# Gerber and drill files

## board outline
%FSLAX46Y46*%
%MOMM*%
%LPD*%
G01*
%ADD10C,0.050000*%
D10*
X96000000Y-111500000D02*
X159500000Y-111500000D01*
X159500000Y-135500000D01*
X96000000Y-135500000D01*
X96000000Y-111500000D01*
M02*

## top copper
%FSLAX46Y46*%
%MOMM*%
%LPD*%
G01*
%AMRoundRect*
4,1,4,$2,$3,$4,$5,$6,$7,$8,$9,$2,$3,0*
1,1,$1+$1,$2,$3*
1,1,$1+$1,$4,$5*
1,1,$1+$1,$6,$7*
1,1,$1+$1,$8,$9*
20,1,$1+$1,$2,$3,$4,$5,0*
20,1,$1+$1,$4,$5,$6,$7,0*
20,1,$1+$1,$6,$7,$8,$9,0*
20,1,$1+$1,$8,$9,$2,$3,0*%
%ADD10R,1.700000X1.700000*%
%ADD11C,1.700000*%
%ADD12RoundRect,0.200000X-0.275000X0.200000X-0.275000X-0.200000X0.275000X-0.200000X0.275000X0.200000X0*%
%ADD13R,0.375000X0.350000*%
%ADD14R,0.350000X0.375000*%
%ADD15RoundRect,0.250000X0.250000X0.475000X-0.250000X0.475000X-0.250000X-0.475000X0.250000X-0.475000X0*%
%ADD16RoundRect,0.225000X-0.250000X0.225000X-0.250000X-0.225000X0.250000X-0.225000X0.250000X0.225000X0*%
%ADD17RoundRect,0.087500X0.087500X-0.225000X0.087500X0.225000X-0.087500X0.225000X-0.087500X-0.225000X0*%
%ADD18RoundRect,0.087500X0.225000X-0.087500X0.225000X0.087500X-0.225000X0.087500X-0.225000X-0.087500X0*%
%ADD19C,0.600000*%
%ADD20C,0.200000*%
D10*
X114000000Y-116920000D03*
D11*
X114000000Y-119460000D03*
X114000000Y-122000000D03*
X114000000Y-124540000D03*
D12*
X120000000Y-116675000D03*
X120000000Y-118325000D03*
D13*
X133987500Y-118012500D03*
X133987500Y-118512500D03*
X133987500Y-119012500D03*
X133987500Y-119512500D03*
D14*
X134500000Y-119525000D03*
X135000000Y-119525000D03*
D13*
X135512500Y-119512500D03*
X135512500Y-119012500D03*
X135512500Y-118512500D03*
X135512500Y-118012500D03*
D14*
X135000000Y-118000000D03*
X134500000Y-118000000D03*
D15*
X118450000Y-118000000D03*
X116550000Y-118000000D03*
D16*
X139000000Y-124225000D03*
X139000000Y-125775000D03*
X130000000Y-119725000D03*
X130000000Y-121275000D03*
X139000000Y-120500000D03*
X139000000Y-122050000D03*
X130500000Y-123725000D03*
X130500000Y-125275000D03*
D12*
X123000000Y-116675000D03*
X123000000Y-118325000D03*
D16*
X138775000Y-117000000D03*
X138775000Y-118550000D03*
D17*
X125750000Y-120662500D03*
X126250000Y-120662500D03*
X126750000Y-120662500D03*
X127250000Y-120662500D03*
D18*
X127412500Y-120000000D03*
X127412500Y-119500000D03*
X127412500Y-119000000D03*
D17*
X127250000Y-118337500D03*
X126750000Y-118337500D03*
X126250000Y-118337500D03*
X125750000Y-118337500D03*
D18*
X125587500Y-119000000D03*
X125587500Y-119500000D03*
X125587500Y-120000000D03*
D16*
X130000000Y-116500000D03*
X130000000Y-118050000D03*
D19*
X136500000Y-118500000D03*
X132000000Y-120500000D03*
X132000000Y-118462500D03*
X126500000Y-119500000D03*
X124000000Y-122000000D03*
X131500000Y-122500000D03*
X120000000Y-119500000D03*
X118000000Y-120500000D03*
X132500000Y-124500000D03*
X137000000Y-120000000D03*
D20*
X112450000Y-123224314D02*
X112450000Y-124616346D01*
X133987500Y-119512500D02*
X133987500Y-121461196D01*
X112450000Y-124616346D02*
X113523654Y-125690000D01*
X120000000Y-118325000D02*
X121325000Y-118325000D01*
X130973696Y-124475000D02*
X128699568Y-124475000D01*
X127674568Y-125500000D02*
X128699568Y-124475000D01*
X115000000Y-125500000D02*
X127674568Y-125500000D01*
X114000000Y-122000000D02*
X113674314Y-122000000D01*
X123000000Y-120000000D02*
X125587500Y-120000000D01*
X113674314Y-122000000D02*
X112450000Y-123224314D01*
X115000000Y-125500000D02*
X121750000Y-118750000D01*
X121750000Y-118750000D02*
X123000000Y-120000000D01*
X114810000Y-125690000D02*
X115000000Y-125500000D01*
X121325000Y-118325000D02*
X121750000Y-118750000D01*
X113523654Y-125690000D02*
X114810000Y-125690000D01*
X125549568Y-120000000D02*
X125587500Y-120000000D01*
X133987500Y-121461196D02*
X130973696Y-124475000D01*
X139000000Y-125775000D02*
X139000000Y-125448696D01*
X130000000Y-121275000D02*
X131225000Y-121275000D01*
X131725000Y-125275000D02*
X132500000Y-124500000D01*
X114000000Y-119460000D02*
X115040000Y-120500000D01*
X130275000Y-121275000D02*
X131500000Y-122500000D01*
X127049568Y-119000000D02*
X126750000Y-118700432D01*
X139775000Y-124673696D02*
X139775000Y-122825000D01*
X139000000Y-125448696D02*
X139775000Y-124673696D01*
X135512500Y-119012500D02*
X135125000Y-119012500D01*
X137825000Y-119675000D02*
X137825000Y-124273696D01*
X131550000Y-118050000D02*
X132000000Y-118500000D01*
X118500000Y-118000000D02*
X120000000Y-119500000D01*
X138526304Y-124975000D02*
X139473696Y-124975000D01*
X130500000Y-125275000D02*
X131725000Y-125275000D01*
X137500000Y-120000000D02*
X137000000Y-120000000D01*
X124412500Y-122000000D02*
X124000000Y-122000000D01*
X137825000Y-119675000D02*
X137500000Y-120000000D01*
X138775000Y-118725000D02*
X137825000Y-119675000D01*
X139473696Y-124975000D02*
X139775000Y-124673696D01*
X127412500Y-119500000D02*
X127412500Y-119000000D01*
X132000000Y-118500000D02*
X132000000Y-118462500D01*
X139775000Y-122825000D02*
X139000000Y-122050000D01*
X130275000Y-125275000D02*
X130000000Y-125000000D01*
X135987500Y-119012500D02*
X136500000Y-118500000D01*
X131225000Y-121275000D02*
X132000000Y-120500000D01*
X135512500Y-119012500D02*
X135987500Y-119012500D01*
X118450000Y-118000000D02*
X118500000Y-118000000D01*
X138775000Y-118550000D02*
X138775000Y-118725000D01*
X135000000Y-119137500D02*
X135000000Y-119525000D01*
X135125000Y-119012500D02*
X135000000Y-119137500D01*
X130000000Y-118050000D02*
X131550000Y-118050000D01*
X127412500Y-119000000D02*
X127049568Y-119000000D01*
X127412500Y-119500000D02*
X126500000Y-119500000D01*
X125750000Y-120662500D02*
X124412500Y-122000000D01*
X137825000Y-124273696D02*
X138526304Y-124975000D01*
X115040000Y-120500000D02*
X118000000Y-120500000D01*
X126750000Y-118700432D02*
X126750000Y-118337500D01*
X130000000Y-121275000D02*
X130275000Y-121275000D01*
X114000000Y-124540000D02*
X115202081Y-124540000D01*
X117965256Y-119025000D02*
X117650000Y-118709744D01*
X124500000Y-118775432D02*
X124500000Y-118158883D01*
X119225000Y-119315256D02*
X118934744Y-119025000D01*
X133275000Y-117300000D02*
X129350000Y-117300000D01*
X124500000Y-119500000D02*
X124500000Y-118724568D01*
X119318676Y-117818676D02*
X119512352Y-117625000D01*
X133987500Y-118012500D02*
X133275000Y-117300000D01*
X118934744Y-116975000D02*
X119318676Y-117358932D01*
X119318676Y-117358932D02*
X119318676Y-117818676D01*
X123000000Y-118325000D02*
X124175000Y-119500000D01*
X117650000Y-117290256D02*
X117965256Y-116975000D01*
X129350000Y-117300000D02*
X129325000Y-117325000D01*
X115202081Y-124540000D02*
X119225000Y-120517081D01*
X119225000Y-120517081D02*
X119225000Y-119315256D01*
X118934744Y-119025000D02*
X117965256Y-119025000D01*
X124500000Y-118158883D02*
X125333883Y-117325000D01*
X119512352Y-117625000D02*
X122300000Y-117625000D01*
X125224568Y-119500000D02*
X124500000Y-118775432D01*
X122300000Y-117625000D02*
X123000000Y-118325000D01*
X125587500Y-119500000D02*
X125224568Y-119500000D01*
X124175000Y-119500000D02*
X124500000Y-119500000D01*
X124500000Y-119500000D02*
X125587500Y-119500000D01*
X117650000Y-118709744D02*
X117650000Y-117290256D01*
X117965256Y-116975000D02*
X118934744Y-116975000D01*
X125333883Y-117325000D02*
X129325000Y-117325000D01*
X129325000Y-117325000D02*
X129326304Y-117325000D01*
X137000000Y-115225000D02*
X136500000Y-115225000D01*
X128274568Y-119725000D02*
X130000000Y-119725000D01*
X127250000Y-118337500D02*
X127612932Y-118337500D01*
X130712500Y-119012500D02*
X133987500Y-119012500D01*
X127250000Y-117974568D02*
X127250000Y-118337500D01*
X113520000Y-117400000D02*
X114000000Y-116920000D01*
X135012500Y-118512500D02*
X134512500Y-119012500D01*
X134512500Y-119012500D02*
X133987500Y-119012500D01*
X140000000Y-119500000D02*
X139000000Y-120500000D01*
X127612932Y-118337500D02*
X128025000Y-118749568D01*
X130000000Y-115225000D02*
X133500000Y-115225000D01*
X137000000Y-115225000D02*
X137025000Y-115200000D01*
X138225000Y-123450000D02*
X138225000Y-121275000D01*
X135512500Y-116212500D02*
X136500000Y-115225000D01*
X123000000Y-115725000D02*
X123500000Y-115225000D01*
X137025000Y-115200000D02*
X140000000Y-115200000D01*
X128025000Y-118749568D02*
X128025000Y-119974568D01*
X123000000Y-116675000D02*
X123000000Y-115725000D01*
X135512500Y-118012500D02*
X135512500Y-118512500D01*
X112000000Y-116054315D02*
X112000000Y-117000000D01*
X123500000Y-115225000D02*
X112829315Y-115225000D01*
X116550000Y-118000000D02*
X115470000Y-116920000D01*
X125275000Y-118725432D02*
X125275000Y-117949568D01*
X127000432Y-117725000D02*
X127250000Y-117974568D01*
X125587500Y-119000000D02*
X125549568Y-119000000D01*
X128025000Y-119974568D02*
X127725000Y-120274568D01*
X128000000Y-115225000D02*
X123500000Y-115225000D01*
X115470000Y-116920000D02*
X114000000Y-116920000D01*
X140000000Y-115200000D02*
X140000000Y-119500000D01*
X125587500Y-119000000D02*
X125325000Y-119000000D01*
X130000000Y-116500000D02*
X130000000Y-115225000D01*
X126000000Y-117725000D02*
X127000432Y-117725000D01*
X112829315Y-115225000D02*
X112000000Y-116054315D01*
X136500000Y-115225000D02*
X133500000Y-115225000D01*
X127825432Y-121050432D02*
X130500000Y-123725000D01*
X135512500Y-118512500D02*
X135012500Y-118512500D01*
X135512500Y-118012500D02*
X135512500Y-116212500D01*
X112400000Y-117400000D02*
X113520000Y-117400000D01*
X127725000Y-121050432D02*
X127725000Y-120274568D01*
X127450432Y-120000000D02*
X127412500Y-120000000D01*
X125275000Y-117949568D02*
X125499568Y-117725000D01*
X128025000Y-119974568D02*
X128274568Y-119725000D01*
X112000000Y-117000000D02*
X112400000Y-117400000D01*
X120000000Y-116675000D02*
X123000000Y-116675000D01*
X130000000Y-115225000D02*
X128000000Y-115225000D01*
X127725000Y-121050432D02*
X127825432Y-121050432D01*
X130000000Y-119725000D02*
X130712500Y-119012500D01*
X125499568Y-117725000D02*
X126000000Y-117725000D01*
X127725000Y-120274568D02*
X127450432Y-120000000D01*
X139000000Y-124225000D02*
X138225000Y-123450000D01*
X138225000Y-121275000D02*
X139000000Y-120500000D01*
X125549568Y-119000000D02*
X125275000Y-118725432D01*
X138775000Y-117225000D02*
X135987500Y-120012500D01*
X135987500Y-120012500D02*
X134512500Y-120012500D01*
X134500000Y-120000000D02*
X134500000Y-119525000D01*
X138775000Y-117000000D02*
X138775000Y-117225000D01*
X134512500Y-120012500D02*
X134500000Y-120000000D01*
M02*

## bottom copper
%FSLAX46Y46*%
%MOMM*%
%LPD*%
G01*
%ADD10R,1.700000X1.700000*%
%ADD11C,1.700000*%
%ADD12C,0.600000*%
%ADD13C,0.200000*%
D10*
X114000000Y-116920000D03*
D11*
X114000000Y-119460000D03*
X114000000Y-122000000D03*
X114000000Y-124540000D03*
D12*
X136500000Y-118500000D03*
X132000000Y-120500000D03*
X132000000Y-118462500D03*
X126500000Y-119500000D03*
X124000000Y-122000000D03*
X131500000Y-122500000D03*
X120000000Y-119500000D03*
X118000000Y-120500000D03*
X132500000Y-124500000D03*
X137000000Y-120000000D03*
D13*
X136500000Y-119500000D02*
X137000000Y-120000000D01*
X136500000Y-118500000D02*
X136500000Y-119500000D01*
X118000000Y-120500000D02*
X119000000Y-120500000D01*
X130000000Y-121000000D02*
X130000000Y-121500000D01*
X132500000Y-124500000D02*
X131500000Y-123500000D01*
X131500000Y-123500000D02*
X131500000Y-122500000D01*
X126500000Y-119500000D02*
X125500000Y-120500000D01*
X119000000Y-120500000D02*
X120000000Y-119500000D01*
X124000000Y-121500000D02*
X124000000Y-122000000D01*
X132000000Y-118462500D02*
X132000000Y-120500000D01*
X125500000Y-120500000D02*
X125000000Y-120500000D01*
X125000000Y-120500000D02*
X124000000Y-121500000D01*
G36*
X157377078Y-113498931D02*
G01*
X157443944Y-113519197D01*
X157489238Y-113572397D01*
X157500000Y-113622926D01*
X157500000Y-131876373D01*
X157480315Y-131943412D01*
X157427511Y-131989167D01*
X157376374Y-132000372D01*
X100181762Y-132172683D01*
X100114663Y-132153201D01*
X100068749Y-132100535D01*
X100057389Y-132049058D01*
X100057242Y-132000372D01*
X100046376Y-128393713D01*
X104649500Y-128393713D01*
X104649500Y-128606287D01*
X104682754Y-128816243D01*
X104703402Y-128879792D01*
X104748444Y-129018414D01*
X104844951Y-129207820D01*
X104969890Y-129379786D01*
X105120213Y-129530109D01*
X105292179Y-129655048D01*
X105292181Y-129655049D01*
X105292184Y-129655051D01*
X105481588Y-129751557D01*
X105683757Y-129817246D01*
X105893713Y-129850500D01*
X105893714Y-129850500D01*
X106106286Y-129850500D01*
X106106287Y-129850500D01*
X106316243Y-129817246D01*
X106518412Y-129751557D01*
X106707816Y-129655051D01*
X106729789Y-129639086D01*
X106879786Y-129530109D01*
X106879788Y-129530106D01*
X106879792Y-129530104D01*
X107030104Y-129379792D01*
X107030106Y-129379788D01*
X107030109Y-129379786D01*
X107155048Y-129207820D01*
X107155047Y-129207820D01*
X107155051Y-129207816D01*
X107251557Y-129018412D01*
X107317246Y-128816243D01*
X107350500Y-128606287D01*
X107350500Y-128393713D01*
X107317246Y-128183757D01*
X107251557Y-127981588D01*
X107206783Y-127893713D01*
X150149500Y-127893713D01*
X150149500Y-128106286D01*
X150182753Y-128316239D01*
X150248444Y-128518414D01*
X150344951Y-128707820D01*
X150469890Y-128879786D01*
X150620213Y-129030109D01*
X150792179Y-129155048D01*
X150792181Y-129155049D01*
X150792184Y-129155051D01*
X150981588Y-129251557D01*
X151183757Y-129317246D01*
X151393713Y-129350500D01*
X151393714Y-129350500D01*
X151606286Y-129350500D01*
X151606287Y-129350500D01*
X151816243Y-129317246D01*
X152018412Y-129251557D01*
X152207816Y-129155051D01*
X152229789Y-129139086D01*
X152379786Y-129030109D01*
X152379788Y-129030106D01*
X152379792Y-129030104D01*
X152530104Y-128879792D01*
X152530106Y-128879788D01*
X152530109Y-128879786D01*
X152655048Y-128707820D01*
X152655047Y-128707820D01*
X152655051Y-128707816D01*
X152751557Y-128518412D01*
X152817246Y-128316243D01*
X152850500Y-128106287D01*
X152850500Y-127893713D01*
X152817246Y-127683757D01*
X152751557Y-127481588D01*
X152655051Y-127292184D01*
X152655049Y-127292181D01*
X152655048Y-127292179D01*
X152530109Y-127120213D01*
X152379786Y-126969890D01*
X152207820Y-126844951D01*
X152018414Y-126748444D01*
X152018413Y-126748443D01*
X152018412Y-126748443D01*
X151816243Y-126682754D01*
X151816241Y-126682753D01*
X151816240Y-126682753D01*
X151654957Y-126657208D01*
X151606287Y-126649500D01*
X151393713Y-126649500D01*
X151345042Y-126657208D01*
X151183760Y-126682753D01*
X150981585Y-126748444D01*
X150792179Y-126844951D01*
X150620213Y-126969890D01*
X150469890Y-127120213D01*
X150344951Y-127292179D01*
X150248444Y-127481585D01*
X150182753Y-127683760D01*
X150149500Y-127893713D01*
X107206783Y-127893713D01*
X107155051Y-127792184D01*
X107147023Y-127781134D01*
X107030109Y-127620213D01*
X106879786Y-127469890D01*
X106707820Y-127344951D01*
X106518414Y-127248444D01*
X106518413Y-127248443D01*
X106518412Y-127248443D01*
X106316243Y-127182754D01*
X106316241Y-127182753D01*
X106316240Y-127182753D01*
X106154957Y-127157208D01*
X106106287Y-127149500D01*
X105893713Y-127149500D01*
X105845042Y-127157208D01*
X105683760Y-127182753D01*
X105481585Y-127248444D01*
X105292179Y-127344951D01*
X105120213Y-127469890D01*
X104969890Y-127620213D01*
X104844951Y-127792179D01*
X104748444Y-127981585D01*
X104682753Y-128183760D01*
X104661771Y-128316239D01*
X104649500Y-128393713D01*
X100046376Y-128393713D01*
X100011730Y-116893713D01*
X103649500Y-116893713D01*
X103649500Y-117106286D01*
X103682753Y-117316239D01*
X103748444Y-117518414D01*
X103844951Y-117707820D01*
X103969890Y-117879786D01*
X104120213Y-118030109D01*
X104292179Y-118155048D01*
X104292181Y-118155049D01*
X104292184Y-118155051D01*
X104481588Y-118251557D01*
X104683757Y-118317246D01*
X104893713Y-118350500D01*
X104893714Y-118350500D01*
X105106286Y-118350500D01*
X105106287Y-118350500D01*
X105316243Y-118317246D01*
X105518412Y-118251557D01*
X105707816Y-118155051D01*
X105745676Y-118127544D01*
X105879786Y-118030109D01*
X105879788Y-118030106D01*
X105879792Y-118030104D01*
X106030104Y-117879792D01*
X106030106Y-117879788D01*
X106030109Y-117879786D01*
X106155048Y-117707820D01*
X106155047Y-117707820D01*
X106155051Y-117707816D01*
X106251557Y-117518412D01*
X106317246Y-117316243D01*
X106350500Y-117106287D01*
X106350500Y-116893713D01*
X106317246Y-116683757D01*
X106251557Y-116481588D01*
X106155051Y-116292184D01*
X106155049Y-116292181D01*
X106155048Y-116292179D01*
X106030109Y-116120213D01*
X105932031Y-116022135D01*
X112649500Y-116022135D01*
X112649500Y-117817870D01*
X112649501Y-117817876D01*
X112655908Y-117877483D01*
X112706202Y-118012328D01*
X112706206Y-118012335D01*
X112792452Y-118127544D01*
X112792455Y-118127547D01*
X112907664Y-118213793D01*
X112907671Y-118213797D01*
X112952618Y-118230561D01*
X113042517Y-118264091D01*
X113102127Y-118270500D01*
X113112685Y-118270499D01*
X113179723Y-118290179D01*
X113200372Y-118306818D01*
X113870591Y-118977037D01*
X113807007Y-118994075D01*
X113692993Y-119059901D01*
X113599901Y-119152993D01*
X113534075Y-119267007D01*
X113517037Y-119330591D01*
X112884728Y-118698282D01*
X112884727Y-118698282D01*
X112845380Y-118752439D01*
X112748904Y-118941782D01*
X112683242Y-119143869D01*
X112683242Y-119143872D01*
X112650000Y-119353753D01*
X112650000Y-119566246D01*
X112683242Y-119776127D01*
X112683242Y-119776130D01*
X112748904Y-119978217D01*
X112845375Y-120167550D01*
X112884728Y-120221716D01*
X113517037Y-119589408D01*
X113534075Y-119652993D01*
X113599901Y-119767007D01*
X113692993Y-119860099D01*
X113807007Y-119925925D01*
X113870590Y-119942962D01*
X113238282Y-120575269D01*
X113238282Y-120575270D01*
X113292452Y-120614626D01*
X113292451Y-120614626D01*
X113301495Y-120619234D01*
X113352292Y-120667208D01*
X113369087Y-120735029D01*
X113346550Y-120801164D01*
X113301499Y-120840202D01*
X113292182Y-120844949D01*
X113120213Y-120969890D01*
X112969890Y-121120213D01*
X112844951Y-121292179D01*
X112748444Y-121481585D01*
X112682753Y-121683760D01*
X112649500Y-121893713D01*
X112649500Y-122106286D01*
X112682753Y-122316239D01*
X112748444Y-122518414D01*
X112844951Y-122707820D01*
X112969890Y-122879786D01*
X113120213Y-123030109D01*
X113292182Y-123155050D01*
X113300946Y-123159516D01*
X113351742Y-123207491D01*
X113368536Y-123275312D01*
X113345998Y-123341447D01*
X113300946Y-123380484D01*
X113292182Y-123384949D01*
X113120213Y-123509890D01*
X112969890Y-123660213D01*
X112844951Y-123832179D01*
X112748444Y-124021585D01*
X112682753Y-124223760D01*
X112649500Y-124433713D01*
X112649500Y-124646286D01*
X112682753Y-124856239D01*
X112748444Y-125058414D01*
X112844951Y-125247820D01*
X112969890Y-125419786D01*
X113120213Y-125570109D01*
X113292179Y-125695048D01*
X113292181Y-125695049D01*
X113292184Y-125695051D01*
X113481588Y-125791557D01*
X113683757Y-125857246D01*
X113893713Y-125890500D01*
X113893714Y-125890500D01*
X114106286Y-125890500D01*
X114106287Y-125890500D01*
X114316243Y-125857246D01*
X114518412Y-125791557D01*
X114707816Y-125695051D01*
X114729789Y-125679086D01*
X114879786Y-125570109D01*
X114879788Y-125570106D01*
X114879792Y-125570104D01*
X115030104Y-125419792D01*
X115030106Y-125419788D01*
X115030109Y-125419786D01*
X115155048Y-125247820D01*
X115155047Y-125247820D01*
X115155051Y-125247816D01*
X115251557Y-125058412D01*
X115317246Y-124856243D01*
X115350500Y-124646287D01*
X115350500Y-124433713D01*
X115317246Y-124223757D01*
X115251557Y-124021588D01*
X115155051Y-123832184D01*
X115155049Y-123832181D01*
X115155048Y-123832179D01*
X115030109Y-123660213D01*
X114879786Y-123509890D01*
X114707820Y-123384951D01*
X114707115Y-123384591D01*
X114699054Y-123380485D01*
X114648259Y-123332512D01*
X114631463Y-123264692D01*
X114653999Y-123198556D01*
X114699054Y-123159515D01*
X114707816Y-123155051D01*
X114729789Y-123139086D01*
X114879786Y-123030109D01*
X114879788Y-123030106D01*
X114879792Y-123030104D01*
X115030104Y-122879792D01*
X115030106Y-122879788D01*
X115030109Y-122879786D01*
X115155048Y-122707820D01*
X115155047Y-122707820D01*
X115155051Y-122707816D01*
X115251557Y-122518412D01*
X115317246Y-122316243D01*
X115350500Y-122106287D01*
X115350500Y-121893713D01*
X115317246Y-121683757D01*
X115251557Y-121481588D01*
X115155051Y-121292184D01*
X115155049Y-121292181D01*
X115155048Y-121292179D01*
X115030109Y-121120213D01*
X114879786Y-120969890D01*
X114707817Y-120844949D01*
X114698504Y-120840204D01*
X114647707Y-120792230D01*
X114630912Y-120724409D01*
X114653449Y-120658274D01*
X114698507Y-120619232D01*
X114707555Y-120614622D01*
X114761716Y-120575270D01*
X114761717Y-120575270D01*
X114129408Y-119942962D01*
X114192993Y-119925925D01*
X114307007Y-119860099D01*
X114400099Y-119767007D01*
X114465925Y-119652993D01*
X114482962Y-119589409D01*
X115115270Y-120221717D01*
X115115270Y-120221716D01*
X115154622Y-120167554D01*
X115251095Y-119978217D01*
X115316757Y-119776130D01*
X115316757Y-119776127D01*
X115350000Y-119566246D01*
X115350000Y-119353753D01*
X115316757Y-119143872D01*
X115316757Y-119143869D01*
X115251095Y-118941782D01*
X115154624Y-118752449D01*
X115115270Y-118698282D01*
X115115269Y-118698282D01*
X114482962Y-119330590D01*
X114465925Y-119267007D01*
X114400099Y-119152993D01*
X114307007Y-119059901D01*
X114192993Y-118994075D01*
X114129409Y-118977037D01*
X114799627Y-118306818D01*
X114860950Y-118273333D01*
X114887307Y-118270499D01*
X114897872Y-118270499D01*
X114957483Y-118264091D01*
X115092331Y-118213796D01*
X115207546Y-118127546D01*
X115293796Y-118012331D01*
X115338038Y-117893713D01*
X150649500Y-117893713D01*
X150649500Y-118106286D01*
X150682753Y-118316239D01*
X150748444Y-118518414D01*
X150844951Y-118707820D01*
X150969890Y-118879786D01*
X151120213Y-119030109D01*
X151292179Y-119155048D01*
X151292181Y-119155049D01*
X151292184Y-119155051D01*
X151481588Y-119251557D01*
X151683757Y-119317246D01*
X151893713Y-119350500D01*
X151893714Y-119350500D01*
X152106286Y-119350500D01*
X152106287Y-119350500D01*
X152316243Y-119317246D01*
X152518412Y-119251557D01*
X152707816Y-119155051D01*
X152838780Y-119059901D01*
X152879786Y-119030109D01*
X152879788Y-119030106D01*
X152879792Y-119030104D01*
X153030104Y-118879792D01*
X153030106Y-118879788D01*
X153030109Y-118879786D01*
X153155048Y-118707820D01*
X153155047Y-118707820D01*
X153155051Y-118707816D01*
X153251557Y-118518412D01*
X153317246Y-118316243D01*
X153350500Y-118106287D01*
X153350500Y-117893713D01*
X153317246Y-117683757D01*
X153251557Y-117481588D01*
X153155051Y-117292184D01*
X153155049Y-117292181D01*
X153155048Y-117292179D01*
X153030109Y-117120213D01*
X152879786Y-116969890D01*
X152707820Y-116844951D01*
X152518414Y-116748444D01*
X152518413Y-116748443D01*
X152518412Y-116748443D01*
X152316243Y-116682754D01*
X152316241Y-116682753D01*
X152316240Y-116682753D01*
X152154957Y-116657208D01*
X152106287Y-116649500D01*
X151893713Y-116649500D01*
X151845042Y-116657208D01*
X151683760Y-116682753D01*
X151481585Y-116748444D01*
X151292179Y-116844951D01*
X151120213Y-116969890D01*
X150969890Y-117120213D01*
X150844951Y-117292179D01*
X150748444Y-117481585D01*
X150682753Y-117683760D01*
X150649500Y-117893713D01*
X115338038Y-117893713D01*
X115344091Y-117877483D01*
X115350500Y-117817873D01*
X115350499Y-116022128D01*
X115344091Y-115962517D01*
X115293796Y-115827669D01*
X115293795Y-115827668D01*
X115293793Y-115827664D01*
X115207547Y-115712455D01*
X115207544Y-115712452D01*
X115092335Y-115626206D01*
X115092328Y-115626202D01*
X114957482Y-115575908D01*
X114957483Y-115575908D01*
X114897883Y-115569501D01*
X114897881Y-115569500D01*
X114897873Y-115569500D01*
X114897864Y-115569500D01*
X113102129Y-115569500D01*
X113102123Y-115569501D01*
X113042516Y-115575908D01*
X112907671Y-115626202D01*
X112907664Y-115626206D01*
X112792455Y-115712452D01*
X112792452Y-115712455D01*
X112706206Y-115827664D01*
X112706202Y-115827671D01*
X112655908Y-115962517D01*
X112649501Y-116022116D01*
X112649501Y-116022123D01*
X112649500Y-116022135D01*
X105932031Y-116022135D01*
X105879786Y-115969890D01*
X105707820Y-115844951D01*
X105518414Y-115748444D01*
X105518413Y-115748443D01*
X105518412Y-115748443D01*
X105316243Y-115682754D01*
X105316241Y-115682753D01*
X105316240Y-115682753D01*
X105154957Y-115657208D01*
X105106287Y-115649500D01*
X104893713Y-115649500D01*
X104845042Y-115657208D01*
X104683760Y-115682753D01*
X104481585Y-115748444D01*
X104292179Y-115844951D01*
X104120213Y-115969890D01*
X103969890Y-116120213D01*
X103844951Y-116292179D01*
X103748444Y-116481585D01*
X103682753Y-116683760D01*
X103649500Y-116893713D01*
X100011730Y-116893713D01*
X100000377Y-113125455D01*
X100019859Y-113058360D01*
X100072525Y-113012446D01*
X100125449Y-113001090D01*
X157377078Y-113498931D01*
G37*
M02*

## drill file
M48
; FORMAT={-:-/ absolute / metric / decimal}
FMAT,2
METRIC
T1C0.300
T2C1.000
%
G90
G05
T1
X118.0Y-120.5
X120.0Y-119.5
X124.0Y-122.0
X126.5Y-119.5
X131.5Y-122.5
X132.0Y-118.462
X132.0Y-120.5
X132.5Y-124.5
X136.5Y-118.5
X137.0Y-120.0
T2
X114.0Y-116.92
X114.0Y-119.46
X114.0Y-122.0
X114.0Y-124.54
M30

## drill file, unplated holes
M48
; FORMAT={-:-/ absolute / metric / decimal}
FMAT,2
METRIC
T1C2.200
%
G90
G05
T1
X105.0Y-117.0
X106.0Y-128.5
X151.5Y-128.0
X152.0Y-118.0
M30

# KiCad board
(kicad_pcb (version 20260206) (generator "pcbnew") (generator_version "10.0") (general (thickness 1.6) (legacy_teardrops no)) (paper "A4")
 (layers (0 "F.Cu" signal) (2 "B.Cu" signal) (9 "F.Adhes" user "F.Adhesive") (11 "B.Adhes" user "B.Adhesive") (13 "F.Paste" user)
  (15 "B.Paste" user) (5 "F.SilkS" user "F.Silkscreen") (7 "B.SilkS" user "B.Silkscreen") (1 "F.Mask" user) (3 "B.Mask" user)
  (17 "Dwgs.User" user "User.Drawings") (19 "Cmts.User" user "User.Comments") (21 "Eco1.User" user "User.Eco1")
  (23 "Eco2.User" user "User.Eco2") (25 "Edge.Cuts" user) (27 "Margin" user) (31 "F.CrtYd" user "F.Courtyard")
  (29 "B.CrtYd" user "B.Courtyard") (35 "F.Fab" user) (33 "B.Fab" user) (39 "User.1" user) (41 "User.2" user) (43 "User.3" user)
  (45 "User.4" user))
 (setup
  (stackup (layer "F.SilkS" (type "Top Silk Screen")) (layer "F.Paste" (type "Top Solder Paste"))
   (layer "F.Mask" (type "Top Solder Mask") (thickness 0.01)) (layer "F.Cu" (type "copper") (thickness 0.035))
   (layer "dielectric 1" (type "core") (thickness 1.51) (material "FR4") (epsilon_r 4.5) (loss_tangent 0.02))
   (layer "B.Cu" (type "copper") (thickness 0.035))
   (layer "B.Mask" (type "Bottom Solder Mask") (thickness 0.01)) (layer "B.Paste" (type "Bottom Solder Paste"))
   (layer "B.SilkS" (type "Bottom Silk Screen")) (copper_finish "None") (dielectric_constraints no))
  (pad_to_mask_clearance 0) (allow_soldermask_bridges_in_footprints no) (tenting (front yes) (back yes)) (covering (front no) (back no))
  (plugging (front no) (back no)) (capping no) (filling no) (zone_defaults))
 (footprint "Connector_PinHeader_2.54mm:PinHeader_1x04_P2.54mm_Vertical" (layer "F.Cu") (at 114 116.92)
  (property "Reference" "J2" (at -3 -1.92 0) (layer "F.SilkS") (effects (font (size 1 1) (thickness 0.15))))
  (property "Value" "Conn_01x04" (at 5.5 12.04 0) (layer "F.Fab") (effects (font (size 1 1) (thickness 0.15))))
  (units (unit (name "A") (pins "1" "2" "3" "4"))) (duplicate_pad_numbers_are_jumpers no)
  (pad "1" thru_hole rect (at 0 0) (size 1.7 1.7) (drill 1) (layers "*.Cu" "*.Mask") (remove_unused_layers no) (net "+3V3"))
  (pad "2" thru_hole circle (at 0 2.54) (size 1.7 1.7) (drill 1) (layers "*.Cu" "*.Mask") (remove_unused_layers no) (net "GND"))
  (pad "3" thru_hole circle (at 0 5.08) (size 1.7 1.7) (drill 1) (layers "*.Cu" "*.Mask") (remove_unused_layers no) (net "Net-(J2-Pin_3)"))
  (pad "4" thru_hole circle (at 0 7.62) (size 1.7 1.7) (drill 1) (layers "*.Cu" "*.Mask") (remove_unused_layers no) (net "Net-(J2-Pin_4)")))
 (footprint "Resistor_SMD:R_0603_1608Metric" (layer "F.Cu") (at 120 117.5 -90)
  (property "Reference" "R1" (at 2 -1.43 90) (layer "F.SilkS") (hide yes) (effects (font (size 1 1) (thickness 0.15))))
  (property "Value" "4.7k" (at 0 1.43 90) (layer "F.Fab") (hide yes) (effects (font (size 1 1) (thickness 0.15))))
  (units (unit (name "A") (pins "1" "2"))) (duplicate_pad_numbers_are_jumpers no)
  (pad "1" smd roundrect (at -0.825 0 270) (size 0.8 0.95) (layers "F.Cu" "F.Mask" "F.Paste") (roundrect_rratio 0.25) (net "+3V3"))
  (pad "2" smd roundrect (at 0.825 0 270) (size 0.8 0.95) (layers "F.Cu" "F.Mask" "F.Paste") (roundrect_rratio 0.25) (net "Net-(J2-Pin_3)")))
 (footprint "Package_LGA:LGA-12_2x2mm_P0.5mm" (layer "F.Cu") (at 134.75 118.7625)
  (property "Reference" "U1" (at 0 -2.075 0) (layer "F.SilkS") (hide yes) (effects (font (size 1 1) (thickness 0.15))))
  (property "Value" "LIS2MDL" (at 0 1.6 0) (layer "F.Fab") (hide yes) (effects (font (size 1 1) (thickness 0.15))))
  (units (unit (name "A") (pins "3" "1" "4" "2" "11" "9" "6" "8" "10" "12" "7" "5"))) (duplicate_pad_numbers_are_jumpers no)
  (pad "1" smd rect (at -0.7625 -0.75) (size 0.375 0.35) (layers "F.Cu" "F.Mask" "F.Paste") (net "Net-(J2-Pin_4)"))
  (pad "2" smd rect (at -0.7625 -0.25) (size 0.375 0.35) (layers "F.Cu" "F.Mask" "F.Paste") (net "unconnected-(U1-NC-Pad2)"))
  (pad "3" smd rect (at -0.7625 0.25) (size 0.375 0.35) (layers "F.Cu" "F.Mask" "F.Paste") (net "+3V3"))
  (pad "4" smd rect (at -0.7625 0.75) (size 0.375 0.35) (layers "F.Cu" "F.Mask" "F.Paste") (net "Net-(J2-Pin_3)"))
  (pad "5" smd rect (at -0.25 0.7625 90) (size 0.375 0.35) (layers "F.Cu" "F.Mask" "F.Paste") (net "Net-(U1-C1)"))
  (pad "6" smd rect (at 0.25 0.7625 90) (size 0.375 0.35) (layers "F.Cu" "F.Mask" "F.Paste") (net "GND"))
  (pad "7" smd rect (at 0.7625 0.75) (size 0.375 0.35) (layers "F.Cu" "F.Mask" "F.Paste") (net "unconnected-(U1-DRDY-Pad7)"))
  (pad "8" smd rect (at 0.7625 0.25) (size 0.375 0.35) (layers "F.Cu" "F.Mask" "F.Paste") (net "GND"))
  (pad "9" smd rect (at 0.7625 -0.25) (size 0.375 0.35) (layers "F.Cu" "F.Mask" "F.Paste") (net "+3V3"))
  (pad "10" smd rect (at 0.7625 -0.75) (size 0.375 0.35) (layers "F.Cu" "F.Mask" "F.Paste") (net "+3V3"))
  (pad "11" smd rect (at 0.25 -0.7625 90) (size 0.375 0.35) (layers "F.Cu" "F.Mask" "F.Paste") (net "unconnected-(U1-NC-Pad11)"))
  (pad "12" smd rect (at -0.25 -0.7625 90) (size 0.375 0.35) (layers "F.Cu" "F.Mask" "F.Paste") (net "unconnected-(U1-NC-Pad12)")))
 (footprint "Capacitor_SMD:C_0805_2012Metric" (layer "F.Cu") (at 117.5 118 180)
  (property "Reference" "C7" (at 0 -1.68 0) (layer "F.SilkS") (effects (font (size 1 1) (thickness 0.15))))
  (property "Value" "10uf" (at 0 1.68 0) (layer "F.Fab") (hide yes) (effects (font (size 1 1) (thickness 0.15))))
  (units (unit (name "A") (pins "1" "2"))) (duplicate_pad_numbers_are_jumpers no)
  (pad "1" smd roundrect (at -0.95 0 180) (size 1 1.45) (layers "F.Cu" "F.Mask" "F.Paste") (roundrect_rratio 0.25) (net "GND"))
  (pad "2" smd roundrect (at 0.95 0 180) (size 1 1.45) (layers "F.Cu" "F.Mask" "F.Paste") (roundrect_rratio 0.25) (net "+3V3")))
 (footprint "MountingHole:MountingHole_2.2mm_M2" (layer "F.Cu") (at 105 117)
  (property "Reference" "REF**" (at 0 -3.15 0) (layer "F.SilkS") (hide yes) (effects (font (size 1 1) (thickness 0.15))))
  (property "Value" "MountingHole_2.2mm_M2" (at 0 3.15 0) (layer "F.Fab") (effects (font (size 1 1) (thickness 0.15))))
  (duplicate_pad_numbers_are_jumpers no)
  (pad "" np_thru_hole circle (at 0 0) (size 2.2 2.2) (drill 2.2) (layers "*.Cu" "*.Mask")))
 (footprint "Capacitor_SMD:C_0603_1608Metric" (layer "F.Cu") (at 139 125 -90)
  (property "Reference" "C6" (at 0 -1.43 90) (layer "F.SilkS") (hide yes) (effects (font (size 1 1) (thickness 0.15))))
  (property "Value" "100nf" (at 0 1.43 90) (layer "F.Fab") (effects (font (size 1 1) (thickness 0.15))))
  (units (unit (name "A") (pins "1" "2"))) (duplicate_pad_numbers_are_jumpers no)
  (pad "1" smd roundrect (at -0.775 0 270) (size 0.9 0.95) (layers "F.Cu" "F.Mask" "F.Paste") (roundrect_rratio 0.25) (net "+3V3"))
  (pad "2" smd roundrect (at 0.775 0 270) (size 0.9 0.95) (layers "F.Cu" "F.Mask" "F.Paste") (roundrect_rratio 0.25) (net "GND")))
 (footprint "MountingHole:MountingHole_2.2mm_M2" (layer "F.Cu") (at 151.5 128)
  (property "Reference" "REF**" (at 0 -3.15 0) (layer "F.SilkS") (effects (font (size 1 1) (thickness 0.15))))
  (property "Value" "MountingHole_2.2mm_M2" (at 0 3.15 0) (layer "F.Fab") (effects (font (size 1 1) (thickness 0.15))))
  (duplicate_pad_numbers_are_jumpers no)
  (pad "" np_thru_hole circle (at 0 0) (size 2.2 2.2) (drill 2.2) (layers "*.Cu" "*.Mask")))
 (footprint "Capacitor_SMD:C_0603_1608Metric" (layer "F.Cu") (at 130 120.5 -90)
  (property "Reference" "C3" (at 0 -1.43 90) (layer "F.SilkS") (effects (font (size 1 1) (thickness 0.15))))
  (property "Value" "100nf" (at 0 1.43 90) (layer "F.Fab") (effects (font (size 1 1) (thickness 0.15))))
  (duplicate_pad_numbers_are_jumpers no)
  (pad "1" smd roundrect (at -0.775 0 270) (size 0.9 0.95) (layers "F.Cu" "F.Mask" "F.Paste") (roundrect_rratio 0.25) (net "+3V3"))
  (pad "2" smd roundrect (at 0.775 0 270) (size 0.9 0.95) (layers "F.Cu" "F.Mask" "F.Paste") (roundrect_rratio 0.25) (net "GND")))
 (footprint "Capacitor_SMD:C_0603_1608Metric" (layer "F.Cu") (at 139 121.275 -90)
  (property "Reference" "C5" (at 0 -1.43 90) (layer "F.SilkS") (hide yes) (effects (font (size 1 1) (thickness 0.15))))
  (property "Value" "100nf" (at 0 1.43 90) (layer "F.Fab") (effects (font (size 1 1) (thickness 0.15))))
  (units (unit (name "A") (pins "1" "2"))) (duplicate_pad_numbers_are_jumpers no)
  (pad "1" smd roundrect (at -0.775 0 270) (size 0.9 0.95) (layers "F.Cu" "F.Mask" "F.Paste") (roundrect_rratio 0.25) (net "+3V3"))
  (pad "2" smd roundrect (at 0.775 0 270) (size 0.9 0.95) (layers "F.Cu" "F.Mask" "F.Paste") (roundrect_rratio 0.25) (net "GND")))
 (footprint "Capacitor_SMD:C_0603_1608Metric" (layer "F.Cu") (at 130.5 124.5 -90)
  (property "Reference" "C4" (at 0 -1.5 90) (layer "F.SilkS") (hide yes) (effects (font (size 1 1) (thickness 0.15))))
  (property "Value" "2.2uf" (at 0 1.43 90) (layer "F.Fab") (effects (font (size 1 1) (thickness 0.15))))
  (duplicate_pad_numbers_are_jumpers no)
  (pad "1" smd roundrect (at -0.775 0 270) (size 0.9 0.95) (layers "F.Cu" "F.Mask" "F.Paste") (roundrect_rratio 0.25) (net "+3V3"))
  (pad "2" smd roundrect (at 0.775 0 270) (size 0.9 0.95) (layers "F.Cu" "F.Mask" "F.Paste") (roundrect_rratio 0.25) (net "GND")))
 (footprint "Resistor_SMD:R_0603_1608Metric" (layer "F.Cu") (at 123 117.5 -90)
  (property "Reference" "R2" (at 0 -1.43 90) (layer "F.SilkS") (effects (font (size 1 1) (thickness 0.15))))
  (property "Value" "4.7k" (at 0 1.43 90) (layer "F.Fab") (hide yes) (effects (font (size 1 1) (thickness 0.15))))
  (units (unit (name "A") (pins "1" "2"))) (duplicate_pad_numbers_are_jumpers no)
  (pad "1" smd roundrect (at -0.825 0 270) (size 0.8 0.95) (layers "F.Cu" "F.Mask" "F.Paste") (roundrect_rratio 0.25) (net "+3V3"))
  (pad "2" smd roundrect (at 0.825 0 270) (size 0.8 0.95) (layers "F.Cu" "F.Mask" "F.Paste") (roundrect_rratio 0.25) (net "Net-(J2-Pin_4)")))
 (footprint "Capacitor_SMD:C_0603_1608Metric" (layer "F.Cu") (at 138.775 117.775 -90)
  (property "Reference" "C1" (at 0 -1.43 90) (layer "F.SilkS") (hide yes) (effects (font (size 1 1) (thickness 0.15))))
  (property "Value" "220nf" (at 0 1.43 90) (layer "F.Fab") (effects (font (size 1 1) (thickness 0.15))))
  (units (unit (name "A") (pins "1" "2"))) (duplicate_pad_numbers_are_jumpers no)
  (pad "1" smd roundrect (at -0.775 0 270) (size 0.9 0.95) (layers "F.Cu" "F.Mask" "F.Paste") (roundrect_rratio 0.25) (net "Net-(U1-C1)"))
  (pad "2" smd roundrect (at 0.775 0 270) (size 0.9 0.95) (layers "F.Cu" "F.Mask" "F.Paste") (roundrect_rratio 0.25) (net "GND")))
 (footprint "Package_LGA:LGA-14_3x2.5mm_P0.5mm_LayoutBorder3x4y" (layer "F.Cu") (at 126.5 119.5 90)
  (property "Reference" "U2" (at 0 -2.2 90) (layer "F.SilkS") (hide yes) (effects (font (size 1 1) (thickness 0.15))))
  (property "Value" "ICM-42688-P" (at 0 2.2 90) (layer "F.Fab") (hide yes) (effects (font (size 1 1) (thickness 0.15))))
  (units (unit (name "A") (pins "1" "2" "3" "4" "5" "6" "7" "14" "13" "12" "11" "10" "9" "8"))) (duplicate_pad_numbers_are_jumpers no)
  (pad "1" smd roundrect (at -1.1625 -0.75 90) (size 0.625 0.35) (layers "F.Cu" "F.Mask" "F.Paste") (roundrect_rratio 0.25) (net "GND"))
  (pad "2" smd roundrect (at -1.1625 -0.25 90) (size 0.625 0.35) (layers "F.Cu" "F.Mask" "F.Paste") (roundrect_rratio 0.25)
   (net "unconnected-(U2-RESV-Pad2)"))
  (pad "3" smd roundrect (at -1.1625 0.25 90) (size 0.625 0.35) (layers "F.Cu" "F.Mask" "F.Paste") (roundrect_rratio 0.25)
   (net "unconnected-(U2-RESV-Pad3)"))
  (pad "4" smd roundrect (at -1.1625 0.75 90) (size 0.625 0.35) (layers "F.Cu" "F.Mask" "F.Paste") (roundrect_rratio 0.25)
   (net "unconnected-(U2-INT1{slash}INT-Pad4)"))
  (pad "5" smd roundrect (at -0.5 0.9125 90) (size 0.35 0.625) (layers "F.Cu" "F.Mask" "F.Paste") (roundrect_rratio 0.25) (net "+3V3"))
  (pad "6" smd roundrect (at 0 0.9125 90) (size 0.35 0.625) (layers "F.Cu" "F.Mask" "F.Paste") (roundrect_rratio 0.25) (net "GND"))
  (pad "7" smd roundrect (at 0.5 0.9125 90) (size 0.35 0.625) (layers "F.Cu" "F.Mask" "F.Paste") (roundrect_rratio 0.25) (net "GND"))
  (pad "8" smd roundrect (at 1.1625 0.75 90) (size 0.625 0.35) (layers "F.Cu" "F.Mask" "F.Paste") (roundrect_rratio 0.25) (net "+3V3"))
  (pad "9" smd roundrect (at 1.1625 0.25 90) (size 0.625 0.35) (layers "F.Cu" "F.Mask" "F.Paste") (roundrect_rratio 0.25) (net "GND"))
  (pad "10" smd roundrect (at 1.1625 -0.25 90) (size 0.625 0.35) (layers "F.Cu" "F.Mask" "F.Paste") (roundrect_rratio 0.25)
   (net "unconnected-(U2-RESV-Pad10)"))
  (pad "11" smd roundrect (at 1.1625 -0.75 90) (size 0.625 0.35) (layers "F.Cu" "F.Mask" "F.Paste") (roundrect_rratio 0.25)
   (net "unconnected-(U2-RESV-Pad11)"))
  (pad "12" smd roundrect (at 0.5 -0.9125 90) (size 0.35 0.625) (layers "F.Cu" "F.Mask" "F.Paste") (roundrect_rratio 0.25) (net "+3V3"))
  (pad "13" smd roundrect (at 0 -0.9125 90) (size 0.35 0.625) (layers "F.Cu" "F.Mask" "F.Paste") (roundrect_rratio 0.25)
   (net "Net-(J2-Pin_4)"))
  (pad "14" smd roundrect (at -0.5 -0.9125 90) (size 0.35 0.625) (layers "F.Cu" "F.Mask" "F.Paste") (roundrect_rratio 0.25)
   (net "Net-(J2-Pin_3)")))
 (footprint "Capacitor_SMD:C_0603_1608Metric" (layer "F.Cu") (at 130 117.275 -90)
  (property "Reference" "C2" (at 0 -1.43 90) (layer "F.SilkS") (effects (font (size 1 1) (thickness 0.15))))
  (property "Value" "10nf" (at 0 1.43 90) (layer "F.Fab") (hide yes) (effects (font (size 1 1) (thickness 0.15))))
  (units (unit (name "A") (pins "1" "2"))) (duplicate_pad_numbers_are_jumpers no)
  (pad "1" smd roundrect (at -0.775 0 270) (size 0.9 0.95) (layers "F.Cu" "F.Mask" "F.Paste") (roundrect_rratio 0.25) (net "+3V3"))
  (pad "2" smd roundrect (at 0.775 0 270) (size 0.9 0.95) (layers "F.Cu" "F.Mask" "F.Paste") (roundrect_rratio 0.25) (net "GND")))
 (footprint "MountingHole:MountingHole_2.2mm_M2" (layer "F.Cu") (at 152 118)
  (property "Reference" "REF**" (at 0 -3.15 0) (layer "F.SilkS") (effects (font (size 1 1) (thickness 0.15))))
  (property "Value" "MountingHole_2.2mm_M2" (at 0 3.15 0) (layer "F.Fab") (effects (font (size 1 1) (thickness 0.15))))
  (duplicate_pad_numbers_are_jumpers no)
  (pad "" np_thru_hole circle (at 0 0) (size 2.2 2.2) (drill 2.2) (layers "*.Cu" "*.Mask")))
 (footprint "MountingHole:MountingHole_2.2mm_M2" (layer "F.Cu") (at 106 128.5)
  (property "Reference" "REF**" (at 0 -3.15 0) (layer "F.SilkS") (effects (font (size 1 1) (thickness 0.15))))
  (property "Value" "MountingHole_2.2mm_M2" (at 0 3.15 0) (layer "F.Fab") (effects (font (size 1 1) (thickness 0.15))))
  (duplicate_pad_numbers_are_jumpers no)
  (pad "" np_thru_hole circle (at 0 0) (size 2.2 2.2) (drill 2.2) (layers "*.Cu" "*.Mask")))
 (gr_rect (start 96 111.5) (end 159.5 135.5) (stroke (width 0.05) (type default)) (fill no) (layer "Edge.Cuts"))
 (segment (start 112.45 123.224314) (end 112.45 124.616346) (width 0.2) (layer "F.Cu") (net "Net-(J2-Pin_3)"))
 (segment (start 133.9875 119.5125) (end 133.9875 121.461196) (width 0.2) (layer "F.Cu") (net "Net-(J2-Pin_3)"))
 (segment (start 112.45 124.616346) (end 113.523654 125.69) (width 0.2) (layer "F.Cu") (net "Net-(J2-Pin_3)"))
 (segment (start 120 118.325) (end 121.325 118.325) (width 0.2) (layer "F.Cu") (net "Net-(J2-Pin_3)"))
 (segment (start 130.973696 124.475) (end 128.699568 124.475) (width 0.2) (layer "F.Cu") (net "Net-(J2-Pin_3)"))
 (segment (start 127.674568 125.5) (end 128.699568 124.475) (width 0.2) (layer "F.Cu") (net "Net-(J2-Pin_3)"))
 (segment (start 115 125.5) (end 127.674568 125.5) (width 0.2) (layer "F.Cu") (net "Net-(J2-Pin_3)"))
 (segment (start 114 122) (end 113.674314 122) (width 0.2) (layer "F.Cu") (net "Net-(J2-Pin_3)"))
 (segment (start 123 120) (end 125.5875 120) (width 0.2) (layer "F.Cu") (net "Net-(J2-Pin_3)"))
 (segment (start 113.674314 122) (end 112.45 123.224314) (width 0.2) (layer "F.Cu") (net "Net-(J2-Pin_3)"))
 (segment (start 115 125.5) (end 121.75 118.75) (width 0.2) (layer "F.Cu") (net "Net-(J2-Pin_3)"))
 (segment (start 121.75 118.75) (end 123 120) (width 0.2) (layer "F.Cu") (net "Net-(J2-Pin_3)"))
 (segment (start 114.81 125.69) (end 115 125.5) (width 0.2) (layer "F.Cu") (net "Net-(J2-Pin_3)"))
 (segment (start 121.325 118.325) (end 121.75 118.75) (width 0.2) (layer "F.Cu") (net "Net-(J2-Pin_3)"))
 (segment (start 113.523654 125.69) (end 114.81 125.69) (width 0.2) (layer "F.Cu") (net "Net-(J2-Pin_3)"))
 (segment (start 125.549568 120) (end 125.5875 120) (width 0.2) (layer "F.Cu") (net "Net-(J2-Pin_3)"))
 (segment (start 133.9875 121.461196) (end 130.973696 124.475) (width 0.2) (layer "F.Cu") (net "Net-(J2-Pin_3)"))
 (segment (start 139 125.775) (end 139 125.448696) (width 0.2) (layer "F.Cu") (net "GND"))
 (segment (start 130 121.275) (end 131.225 121.275) (width 0.2) (layer "F.Cu") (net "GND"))
 (segment (start 131.725 125.275) (end 132.5 124.5) (width 0.2) (layer "F.Cu") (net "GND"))
 (segment (start 114 119.46) (end 115.04 120.5) (width 0.2) (layer "F.Cu") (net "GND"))
 (segment (start 130.275 121.275) (end 131.5 122.5) (width 0.2) (layer "F.Cu") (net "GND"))
 (segment (start 127.049568 119) (end 126.75 118.700432) (width 0.2) (layer "F.Cu") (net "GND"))
 (segment (start 139.775 124.673696) (end 139.775 122.825) (width 0.2) (layer "F.Cu") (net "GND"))
 (segment (start 139 125.448696) (end 139.775 124.673696) (width 0.2) (layer "F.Cu") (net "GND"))
 (segment (start 135.5125 119.0125) (end 135.125 119.0125) (width 0.2) (layer "F.Cu") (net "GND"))
 (segment (start 137.825 119.675) (end 137.825 124.273696) (width 0.2) (layer "F.Cu") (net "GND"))
 (segment (start 131.55 118.05) (end 132 118.5) (width 0.2) (layer "F.Cu") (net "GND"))
 (segment (start 118.5 118) (end 120 119.5) (width 0.2) (layer "F.Cu") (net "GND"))
 (segment (start 138.526304 124.975) (end 139.473696 124.975) (width 0.2) (layer "F.Cu") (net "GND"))
 (segment (start 130.5 125.275) (end 131.725 125.275) (width 0.2) (layer "F.Cu") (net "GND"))
 (segment (start 137.5 120) (end 137 120) (width 0.2) (layer "F.Cu") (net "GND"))
 (segment (start 124.4125 122) (end 124 122) (width 0.2) (layer "F.Cu") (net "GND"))
 (segment (start 137.825 119.675) (end 137.5 120) (width 0.2) (layer "F.Cu") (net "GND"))
 (segment (start 138.775 118.725) (end 137.825 119.675) (width 0.2) (layer "F.Cu") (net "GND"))
 (segment (start 139.473696 124.975) (end 139.775 124.673696) (width 0.2) (layer "F.Cu") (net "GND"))
 (segment (start 127.4125 119.5) (end 127.4125 119) (width 0.2) (layer "F.Cu") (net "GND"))
 (segment (start 132 118.5) (end 132 118.4625) (width 0.2) (layer "F.Cu") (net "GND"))
 (segment (start 139.775 122.825) (end 139 122.05) (width 0.2) (layer "F.Cu") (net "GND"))
 (segment (start 130.275 125.275) (end 130 125) (width 0.2) (layer "F.Cu") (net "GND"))
 (segment (start 135.9875 119.0125) (end 136.5 118.5) (width 0.2) (layer "F.Cu") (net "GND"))
 (segment (start 131.225 121.275) (end 132 120.5) (width 0.2) (layer "F.Cu") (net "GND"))
 (segment (start 135.5125 119.0125) (end 135.9875 119.0125) (width 0.2) (layer "F.Cu") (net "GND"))
 (segment (start 118.45 118) (end 118.5 118) (width 0.2) (layer "F.Cu") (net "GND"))
 (segment (start 138.775 118.55) (end 138.775 118.725) (width 0.2) (layer "F.Cu") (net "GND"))
 (segment (start 135 119.1375) (end 135 119.525) (width 0.2) (layer "F.Cu") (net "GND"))
 (segment (start 135.125 119.0125) (end 135 119.1375) (width 0.2) (layer "F.Cu") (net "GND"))
 (segment (start 130 118.05) (end 131.55 118.05) (width 0.2) (layer "F.Cu") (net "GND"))
 (segment (start 127.4125 119) (end 127.049568 119) (width 0.2) (layer "F.Cu") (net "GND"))
 (segment (start 127.4125 119.5) (end 126.5 119.5) (width 0.2) (layer "F.Cu") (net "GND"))
 (segment (start 125.75 120.6625) (end 124.4125 122) (width 0.2) (layer "F.Cu") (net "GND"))
 (segment (start 137.825 124.273696) (end 138.526304 124.975) (width 0.2) (layer "F.Cu") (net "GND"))
 (segment (start 115.04 120.5) (end 118 120.5) (width 0.2) (layer "F.Cu") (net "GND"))
 (segment (start 126.75 118.700432) (end 126.75 118.3375) (width 0.2) (layer "F.Cu") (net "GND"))
 (segment (start 130 121.275) (end 130.275 121.275) (width 0.2) (layer "F.Cu") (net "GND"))
 (via (at 136.5 118.5) (size 0.6) (drill 0.3) (layers "F.Cu" "B.Cu") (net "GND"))
 (via (at 132 120.5) (size 0.6) (drill 0.3) (layers "F.Cu" "B.Cu") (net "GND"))
 (via (at 132 118.4625) (size 0.6) (drill 0.3) (layers "F.Cu" "B.Cu") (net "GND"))
 (via (at 126.5 119.5) (size 0.6) (drill 0.3) (layers "F.Cu" "B.Cu") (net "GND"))
 (via (at 124 122) (size 0.6) (drill 0.3) (layers "F.Cu" "B.Cu") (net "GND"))
 (via (at 131.5 122.5) (size 0.6) (drill 0.3) (layers "F.Cu" "B.Cu") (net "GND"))
 (via (at 120 119.5) (size 0.6) (drill 0.3) (layers "F.Cu" "B.Cu") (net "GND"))
 (via (at 118 120.5) (size 0.6) (drill 0.3) (layers "F.Cu" "B.Cu") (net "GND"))
 (via (at 132.5 124.5) (size 0.6) (drill 0.3) (layers "F.Cu" "B.Cu") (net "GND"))
 (via (at 137 120) (size 0.6) (drill 0.3) (layers "F.Cu" "B.Cu") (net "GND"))
 (segment (start 136.5 119.5) (end 137 120) (width 0.2) (layer "B.Cu") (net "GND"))
 (segment (start 136.5 118.5) (end 136.5 119.5) (width 0.2) (layer "B.Cu") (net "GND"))
 (segment (start 118 120.5) (end 119 120.5) (width 0.2) (layer "B.Cu") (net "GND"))
 (segment (start 130 121) (end 130 121.5) (width 0.2) (layer "B.Cu") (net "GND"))
 (segment (start 132.5 124.5) (end 131.5 123.5) (width 0.2) (layer "B.Cu") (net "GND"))
 (segment (start 131.5 123.5) (end 131.5 122.5) (width 0.2) (layer "B.Cu") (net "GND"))
 (segment (start 126.5 119.5) (end 125.5 120.5) (width 0.2) (layer "B.Cu") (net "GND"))
 (segment (start 119 120.5) (end 120 119.5) (width 0.2) (layer "B.Cu") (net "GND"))
 (segment (start 124 121.5) (end 124 122) (width 0.2) (layer "B.Cu") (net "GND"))
 (segment (start 132 118.4625) (end 132 120.5) (width 0.2) (layer "B.Cu") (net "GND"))
 (segment (start 125.5 120.5) (end 125 120.5) (width 0.2) (layer "B.Cu") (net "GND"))
 (segment (start 125 120.5) (end 124 121.5) (width 0.2) (layer "B.Cu") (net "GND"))
 (segment (start 114 124.54) (end 115.202081 124.54) (width 0.2) (layer "F.Cu") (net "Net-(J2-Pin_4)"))
 (segment (start 117.965256 119.025) (end 117.65 118.709744) (width 0.2) (layer "F.Cu") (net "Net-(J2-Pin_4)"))
 (segment (start 124.5 118.775432) (end 124.5 118.158883) (width 0.2) (layer "F.Cu") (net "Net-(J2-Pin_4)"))
 (segment (start 119.225 119.315256) (end 118.934744 119.025) (width 0.2) (layer "F.Cu") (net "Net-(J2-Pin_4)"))
 (segment (start 133.275 117.3) (end 129.35 117.3) (width 0.2) (layer "F.Cu") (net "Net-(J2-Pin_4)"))
 (segment (start 124.5 119.5) (end 124.5 118.724568) (width 0.2) (layer "F.Cu") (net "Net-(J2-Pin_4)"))
 (segment (start 119.318676 117.818676) (end 119.512352 117.625) (width 0.2) (layer "F.Cu") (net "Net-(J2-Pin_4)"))
 (segment (start 133.9875 118.0125) (end 133.275 117.3) (width 0.2) (layer "F.Cu") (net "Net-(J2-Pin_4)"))
 (segment (start 118.934744 116.975) (end 119.318676 117.358932) (width 0.2) (layer "F.Cu") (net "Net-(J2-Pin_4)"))
 (segment (start 119.318676 117.358932) (end 119.318676 117.818676) (width 0.2) (layer "F.Cu") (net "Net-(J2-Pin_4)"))
 (segment (start 123 118.325) (end 124.175 119.5) (width 0.2) (layer "F.Cu") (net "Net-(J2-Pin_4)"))
 (segment (start 117.65 117.290256) (end 117.965256 116.975) (width 0.2) (layer "F.Cu") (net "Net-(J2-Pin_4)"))
 (segment (start 129.35 117.3) (end 129.325 117.325) (width 0.2) (layer "F.Cu") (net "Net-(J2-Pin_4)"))
 (segment (start 115.202081 124.54) (end 119.225 120.517081) (width 0.2) (layer "F.Cu") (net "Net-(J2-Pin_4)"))
 (segment (start 119.225 120.517081) (end 119.225 119.315256) (width 0.2) (layer "F.Cu") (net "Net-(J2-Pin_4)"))
 (segment (start 118.934744 119.025) (end 117.965256 119.025) (width 0.2) (layer "F.Cu") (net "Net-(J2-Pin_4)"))
 (segment (start 124.5 118.158883) (end 125.333883 117.325) (width 0.2) (layer "F.Cu") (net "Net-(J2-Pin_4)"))
 (segment (start 119.512352 117.625) (end 122.3 117.625) (width 0.2) (layer "F.Cu") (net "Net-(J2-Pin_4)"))
 (segment (start 125.224568 119.5) (end 124.5 118.775432) (width 0.2) (layer "F.Cu") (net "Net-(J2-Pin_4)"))
 (segment (start 122.3 117.625) (end 123 118.325) (width 0.2) (layer "F.Cu") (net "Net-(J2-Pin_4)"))
 (segment (start 125.5875 119.5) (end 125.224568 119.5) (width 0.2) (layer "F.Cu") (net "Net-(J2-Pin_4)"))
 (segment (start 124.175 119.5) (end 124.5 119.5) (width 0.2) (layer "F.Cu") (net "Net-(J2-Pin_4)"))
 (segment (start 124.5 119.5) (end 125.5875 119.5) (width 0.2) (layer "F.Cu") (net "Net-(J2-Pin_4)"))
 (segment (start 117.65 118.709744) (end 117.65 117.290256) (width 0.2) (layer "F.Cu") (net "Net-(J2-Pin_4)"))
 (segment (start 117.965256 116.975) (end 118.934744 116.975) (width 0.2) (layer "F.Cu") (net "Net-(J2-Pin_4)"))
 (segment (start 125.333883 117.325) (end 129.325 117.325) (width 0.2) (layer "F.Cu") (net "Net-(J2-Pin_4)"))
 (segment (start 129.325 117.325) (end 129.326304 117.325) (width 0.2) (layer "F.Cu") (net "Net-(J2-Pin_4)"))
 (segment (start 137 115.225) (end 136.5 115.225) (width 0.2) (layer "F.Cu") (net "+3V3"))
 (segment (start 128.274568 119.725) (end 130 119.725) (width 0.2) (layer "F.Cu") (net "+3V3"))
 (segment (start 127.25 118.3375) (end 127.612932 118.3375) (width 0.2) (layer "F.Cu") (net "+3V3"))
 (segment (start 130.7125 119.0125) (end 133.9875 119.0125) (width 0.2) (layer "F.Cu") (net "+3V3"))
 (segment (start 127.25 117.974568) (end 127.25 118.3375) (width 0.2) (layer "F.Cu") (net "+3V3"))
 (segment (start 113.52 117.4) (end 114 116.92) (width 0.2) (layer "F.Cu") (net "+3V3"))
 (segment (start 135.0125 118.5125) (end 134.5125 119.0125) (width 0.2) (layer "F.Cu") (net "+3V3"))
 (segment (start 134.5125 119.0125) (end 133.9875 119.0125) (width 0.2) (layer "F.Cu") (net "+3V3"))
 (segment (start 140 119.5) (end 139 120.5) (width 0.2) (layer "F.Cu") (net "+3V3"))
 (segment (start 127.612932 118.3375) (end 128.025 118.749568) (width 0.2) (layer "F.Cu") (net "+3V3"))
 (segment (start 130 115.225) (end 133.5 115.225) (width 0.2) (layer "F.Cu") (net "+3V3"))
 (segment (start 137 115.225) (end 137.025 115.2) (width 0.2) (layer "F.Cu") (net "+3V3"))
 (segment (start 138.225 123.45) (end 138.225 121.275) (width 0.2) (layer "F.Cu") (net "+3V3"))
 (segment (start 135.5125 116.2125) (end 136.5 115.225) (width 0.2) (layer "F.Cu") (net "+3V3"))
 (segment (start 123 115.725) (end 123.5 115.225) (width 0.2) (layer "F.Cu") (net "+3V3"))
 (segment (start 137.025 115.2) (end 140 115.2) (width 0.2) (layer "F.Cu") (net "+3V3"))
 (segment (start 128.025 118.749568) (end 128.025 119.974568) (width 0.2) (layer "F.Cu") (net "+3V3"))
 (segment (start 123 116.675) (end 123 115.725) (width 0.2) (layer "F.Cu") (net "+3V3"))
 (segment (start 135.5125 118.0125) (end 135.5125 118.5125) (width 0.2) (layer "F.Cu") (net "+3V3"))
 (segment (start 112 116.054315) (end 112 117) (width 0.2) (layer "F.Cu") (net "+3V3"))
 (segment (start 123.5 115.225) (end 112.829315 115.225) (width 0.2) (layer "F.Cu") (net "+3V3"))
 (segment (start 116.55 118) (end 115.47 116.92) (width 0.2) (layer "F.Cu") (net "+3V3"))
 (segment (start 125.275 118.725432) (end 125.275 117.949568) (width 0.2) (layer "F.Cu") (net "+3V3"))
 (segment (start 127.000432 117.725) (end 127.25 117.974568) (width 0.2) (layer "F.Cu") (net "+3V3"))
 (segment (start 125.5875 119) (end 125.549568 119) (width 0.2) (layer "F.Cu") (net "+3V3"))
 (segment (start 128.025 119.974568) (end 127.725 120.274568) (width 0.2) (layer "F.Cu") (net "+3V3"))
 (segment (start 128 115.225) (end 123.5 115.225) (width 0.2) (layer "F.Cu") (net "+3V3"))
 (segment (start 115.47 116.92) (end 114 116.92) (width 0.2) (layer "F.Cu") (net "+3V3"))
 (segment (start 140 115.2) (end 140 119.5) (width 0.2) (layer "F.Cu") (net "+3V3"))
 (segment (start 125.5875 119) (end 125.325 119) (width 0.2) (layer "F.Cu") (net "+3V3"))
 (segment (start 130 116.5) (end 130 115.225) (width 0.2) (layer "F.Cu") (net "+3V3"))
 (segment (start 126 117.725) (end 127.000432 117.725) (width 0.2) (layer "F.Cu") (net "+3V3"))
 (segment (start 112.829315 115.225) (end 112 116.054315) (width 0.2) (layer "F.Cu") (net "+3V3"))
 (segment (start 136.5 115.225) (end 133.5 115.225) (width 0.2) (layer "F.Cu") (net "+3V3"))
 (segment (start 127.825432 121.050432) (end 130.5 123.725) (width 0.2) (layer "F.Cu") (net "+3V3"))
 (segment (start 135.5125 118.5125) (end 135.0125 118.5125) (width 0.2) (layer "F.Cu") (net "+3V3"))
 (segment (start 135.5125 118.0125) (end 135.5125 116.2125) (width 0.2) (layer "F.Cu") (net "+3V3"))
 (segment (start 112.4 117.4) (end 113.52 117.4) (width 0.2) (layer "F.Cu") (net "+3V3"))
 (segment (start 127.725 121.050432) (end 127.725 120.274568) (width 0.2) (layer "F.Cu") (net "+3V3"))
 (segment (start 127.450432 120) (end 127.4125 120) (width 0.2) (layer "F.Cu") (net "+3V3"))
 (segment (start 125.275 117.949568) (end 125.499568 117.725) (width 0.2) (layer "F.Cu") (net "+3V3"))
 (segment (start 128.025 119.974568) (end 128.274568 119.725) (width 0.2) (layer "F.Cu") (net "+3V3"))
 (segment (start 112 117) (end 112.4 117.4) (width 0.2) (layer "F.Cu") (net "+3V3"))
 (segment (start 120 116.675) (end 123 116.675) (width 0.2) (layer "F.Cu") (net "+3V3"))
 (segment (start 130 115.225) (end 128 115.225) (width 0.2) (layer "F.Cu") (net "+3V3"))
 (segment (start 127.725 121.050432) (end 127.825432 121.050432) (width 0.2) (layer "F.Cu") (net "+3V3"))
 (segment (start 130 119.725) (end 130.7125 119.0125) (width 0.2) (layer "F.Cu") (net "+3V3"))
 (segment (start 125.499568 117.725) (end 126 117.725) (width 0.2) (layer "F.Cu") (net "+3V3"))
 (segment (start 127.725 120.274568) (end 127.450432 120) (width 0.2) (layer "F.Cu") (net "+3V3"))
 (segment (start 139 124.225) (end 138.225 123.45) (width 0.2) (layer "F.Cu") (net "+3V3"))
 (segment (start 138.225 121.275) (end 139 120.5) (width 0.2) (layer "F.Cu") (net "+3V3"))
 (segment (start 125.549568 119) (end 125.275 118.725432) (width 0.2) (layer "F.Cu") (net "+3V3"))
 (segment (start 138.775 117.225) (end 135.9875 120.0125) (width 0.2) (layer "F.Cu") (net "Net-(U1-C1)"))
 (segment (start 135.9875 120.0125) (end 134.5125 120.0125) (width 0.2) (layer "F.Cu") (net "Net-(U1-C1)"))
 (segment (start 134.5 120) (end 134.5 119.525) (width 0.2) (layer "F.Cu") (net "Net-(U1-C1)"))
 (segment (start 138.775 117) (end 138.775 117.225) (width 0.2) (layer "F.Cu") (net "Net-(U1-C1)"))
 (segment (start 134.5125 120.0125) (end 134.5 120) (width 0.2) (layer "F.Cu") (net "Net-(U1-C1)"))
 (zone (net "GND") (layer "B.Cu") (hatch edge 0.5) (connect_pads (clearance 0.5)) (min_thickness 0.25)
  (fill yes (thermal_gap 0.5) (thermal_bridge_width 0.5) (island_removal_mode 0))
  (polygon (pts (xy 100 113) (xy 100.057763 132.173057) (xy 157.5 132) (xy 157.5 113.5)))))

